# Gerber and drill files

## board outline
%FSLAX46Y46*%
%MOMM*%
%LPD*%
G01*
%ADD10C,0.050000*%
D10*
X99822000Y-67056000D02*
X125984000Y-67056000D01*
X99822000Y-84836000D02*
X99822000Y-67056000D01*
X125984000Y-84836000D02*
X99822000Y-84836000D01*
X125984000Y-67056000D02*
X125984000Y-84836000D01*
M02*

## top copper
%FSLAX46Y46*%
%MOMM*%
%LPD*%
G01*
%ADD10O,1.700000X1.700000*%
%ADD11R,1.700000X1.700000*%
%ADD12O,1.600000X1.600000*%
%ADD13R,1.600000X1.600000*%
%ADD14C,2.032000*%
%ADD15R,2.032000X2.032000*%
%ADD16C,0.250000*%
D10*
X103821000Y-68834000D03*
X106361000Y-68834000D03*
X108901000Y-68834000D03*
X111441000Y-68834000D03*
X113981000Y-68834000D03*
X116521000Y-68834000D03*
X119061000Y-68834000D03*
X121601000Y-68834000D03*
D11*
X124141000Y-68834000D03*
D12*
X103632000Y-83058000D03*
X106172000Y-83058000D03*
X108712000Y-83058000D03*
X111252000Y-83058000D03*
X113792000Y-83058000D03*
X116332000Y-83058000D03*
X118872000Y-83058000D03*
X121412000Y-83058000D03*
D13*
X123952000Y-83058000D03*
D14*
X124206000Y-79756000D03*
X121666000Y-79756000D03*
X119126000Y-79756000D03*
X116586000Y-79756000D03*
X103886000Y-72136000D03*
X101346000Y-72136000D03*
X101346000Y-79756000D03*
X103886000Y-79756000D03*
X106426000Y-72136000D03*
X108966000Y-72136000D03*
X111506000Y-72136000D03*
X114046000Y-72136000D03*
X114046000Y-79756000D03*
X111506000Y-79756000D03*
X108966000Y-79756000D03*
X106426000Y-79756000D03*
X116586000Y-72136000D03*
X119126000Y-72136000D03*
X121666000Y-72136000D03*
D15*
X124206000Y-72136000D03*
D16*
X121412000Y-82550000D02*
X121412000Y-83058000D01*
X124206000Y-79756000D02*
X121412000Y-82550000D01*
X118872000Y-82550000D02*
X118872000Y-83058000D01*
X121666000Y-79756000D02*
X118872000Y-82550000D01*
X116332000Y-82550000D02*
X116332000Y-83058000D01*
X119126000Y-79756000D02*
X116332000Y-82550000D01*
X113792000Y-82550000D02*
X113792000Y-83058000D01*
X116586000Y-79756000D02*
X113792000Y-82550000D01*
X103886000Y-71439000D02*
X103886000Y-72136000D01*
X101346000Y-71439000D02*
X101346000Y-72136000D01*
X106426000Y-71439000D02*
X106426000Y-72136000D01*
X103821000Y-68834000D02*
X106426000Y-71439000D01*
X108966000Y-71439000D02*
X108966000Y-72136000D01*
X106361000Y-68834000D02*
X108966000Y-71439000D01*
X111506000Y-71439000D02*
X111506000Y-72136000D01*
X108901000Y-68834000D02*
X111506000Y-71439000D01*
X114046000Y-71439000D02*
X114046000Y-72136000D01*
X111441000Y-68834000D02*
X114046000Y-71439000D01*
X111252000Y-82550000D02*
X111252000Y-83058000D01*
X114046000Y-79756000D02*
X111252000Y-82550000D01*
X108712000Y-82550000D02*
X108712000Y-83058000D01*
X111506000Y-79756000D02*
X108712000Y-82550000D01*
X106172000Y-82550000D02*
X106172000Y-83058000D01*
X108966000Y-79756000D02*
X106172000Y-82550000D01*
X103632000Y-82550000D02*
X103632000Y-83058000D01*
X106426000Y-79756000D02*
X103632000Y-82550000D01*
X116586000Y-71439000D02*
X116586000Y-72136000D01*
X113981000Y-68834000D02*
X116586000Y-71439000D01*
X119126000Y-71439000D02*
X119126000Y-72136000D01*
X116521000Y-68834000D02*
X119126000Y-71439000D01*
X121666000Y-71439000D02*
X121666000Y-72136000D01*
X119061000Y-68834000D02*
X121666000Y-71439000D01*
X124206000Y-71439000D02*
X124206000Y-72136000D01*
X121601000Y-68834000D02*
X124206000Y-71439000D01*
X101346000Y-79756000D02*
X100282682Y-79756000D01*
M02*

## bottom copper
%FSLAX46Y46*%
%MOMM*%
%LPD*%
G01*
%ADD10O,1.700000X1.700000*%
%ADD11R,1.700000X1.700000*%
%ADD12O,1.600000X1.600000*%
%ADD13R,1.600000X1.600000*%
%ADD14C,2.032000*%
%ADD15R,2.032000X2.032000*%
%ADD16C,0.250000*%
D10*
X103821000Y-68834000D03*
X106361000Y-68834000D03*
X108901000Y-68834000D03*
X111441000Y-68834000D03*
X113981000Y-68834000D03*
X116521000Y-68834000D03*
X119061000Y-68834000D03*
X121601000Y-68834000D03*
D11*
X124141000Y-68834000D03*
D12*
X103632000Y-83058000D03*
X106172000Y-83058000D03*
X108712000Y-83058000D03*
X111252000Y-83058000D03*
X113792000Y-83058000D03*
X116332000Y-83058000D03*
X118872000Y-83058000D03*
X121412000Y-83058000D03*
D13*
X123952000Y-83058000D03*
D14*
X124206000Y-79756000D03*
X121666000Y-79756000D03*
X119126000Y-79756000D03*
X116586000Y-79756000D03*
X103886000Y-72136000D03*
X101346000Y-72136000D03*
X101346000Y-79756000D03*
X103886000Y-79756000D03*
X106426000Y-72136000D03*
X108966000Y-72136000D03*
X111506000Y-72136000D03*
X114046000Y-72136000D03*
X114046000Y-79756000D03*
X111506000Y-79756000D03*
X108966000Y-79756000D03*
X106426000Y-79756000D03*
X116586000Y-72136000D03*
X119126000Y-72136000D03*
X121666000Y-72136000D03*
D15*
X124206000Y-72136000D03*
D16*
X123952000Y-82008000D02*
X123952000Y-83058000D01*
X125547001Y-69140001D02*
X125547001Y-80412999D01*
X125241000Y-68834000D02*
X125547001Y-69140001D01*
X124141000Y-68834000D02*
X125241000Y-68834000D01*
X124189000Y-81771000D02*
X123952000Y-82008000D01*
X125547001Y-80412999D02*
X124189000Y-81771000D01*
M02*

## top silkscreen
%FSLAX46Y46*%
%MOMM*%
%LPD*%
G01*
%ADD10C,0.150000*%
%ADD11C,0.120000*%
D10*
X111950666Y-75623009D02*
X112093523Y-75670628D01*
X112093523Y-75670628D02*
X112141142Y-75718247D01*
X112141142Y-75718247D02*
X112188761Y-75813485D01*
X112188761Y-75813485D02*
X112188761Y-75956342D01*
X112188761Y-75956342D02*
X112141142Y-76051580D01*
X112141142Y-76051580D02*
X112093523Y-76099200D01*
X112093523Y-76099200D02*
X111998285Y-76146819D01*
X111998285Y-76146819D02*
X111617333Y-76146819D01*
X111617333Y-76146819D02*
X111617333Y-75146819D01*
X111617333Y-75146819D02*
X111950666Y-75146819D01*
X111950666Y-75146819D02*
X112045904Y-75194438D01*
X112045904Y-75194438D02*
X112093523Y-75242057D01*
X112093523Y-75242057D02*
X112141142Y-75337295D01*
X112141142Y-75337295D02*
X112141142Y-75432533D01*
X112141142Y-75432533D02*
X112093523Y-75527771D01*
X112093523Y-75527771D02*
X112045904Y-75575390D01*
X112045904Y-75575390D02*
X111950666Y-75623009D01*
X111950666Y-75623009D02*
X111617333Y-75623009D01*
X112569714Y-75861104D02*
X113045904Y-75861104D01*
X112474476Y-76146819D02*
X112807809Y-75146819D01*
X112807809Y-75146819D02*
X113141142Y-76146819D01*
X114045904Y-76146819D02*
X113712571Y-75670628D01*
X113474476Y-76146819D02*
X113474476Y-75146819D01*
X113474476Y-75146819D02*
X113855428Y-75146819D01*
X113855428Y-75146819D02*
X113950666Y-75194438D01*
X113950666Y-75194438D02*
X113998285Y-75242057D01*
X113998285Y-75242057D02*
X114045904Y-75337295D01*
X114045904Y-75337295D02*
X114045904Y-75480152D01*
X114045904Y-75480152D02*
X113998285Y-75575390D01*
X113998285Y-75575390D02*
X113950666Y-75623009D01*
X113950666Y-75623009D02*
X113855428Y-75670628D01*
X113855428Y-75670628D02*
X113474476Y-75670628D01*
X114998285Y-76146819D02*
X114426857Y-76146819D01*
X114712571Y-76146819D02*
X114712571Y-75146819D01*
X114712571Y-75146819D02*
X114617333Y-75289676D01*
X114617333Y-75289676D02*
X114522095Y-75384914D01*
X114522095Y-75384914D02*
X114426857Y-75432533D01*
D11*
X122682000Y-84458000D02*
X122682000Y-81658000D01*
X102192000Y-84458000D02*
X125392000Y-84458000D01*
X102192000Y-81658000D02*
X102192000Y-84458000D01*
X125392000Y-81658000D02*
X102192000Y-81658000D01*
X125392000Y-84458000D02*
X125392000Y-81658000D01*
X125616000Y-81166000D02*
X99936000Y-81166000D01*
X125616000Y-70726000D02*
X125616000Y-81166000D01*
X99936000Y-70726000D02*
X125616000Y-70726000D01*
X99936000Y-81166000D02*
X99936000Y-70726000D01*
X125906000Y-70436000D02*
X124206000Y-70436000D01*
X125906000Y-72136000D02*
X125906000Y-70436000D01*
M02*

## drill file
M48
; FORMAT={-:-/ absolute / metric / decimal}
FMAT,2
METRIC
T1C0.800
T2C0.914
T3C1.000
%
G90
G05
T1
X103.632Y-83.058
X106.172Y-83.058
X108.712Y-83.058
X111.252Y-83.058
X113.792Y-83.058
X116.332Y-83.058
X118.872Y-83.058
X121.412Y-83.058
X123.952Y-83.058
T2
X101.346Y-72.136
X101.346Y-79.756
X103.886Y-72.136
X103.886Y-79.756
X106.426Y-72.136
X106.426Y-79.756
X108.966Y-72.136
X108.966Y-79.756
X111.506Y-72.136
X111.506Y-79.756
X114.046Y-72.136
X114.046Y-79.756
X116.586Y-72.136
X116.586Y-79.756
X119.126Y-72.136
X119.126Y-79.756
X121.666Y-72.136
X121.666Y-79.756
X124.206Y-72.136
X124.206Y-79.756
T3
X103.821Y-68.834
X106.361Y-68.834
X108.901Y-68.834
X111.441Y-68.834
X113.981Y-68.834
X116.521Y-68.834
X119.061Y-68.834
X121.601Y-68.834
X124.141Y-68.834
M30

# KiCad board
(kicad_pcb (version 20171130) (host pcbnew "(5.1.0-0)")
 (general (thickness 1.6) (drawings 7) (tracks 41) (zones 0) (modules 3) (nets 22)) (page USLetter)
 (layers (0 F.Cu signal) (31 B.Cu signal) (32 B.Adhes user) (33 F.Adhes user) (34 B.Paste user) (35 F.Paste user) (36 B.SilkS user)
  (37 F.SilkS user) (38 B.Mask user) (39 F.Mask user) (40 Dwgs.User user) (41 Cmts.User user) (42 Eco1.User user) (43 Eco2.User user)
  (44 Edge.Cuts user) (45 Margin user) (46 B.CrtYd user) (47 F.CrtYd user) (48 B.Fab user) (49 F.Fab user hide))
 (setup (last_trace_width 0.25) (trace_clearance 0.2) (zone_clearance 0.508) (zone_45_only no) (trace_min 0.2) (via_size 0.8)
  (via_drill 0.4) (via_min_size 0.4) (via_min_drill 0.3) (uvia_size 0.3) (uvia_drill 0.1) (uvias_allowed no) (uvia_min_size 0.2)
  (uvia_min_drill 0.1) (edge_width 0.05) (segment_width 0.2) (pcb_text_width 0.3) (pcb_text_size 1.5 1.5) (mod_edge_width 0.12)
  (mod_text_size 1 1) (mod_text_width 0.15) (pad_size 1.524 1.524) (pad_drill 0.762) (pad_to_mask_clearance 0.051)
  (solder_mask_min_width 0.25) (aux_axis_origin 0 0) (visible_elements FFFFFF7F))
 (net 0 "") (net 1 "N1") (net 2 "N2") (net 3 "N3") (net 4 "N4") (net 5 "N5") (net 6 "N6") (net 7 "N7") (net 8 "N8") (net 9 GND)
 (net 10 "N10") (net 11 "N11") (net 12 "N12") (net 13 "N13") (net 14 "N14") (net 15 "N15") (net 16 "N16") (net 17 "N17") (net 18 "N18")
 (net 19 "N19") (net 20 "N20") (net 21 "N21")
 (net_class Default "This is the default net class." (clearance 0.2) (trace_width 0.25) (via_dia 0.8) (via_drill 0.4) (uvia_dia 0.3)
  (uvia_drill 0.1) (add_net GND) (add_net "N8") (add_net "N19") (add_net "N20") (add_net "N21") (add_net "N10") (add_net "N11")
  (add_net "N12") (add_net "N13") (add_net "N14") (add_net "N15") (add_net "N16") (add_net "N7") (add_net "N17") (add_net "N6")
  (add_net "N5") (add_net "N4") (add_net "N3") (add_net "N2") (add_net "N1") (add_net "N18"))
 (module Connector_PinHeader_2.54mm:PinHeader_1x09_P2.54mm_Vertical (layer B.Cu) (at 124.141 68.834 90)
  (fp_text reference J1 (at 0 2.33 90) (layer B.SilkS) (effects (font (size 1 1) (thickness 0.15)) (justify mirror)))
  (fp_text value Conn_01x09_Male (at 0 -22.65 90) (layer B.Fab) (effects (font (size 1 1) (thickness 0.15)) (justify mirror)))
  (pad 9 thru_hole oval (at 0 -20.32 90) (size 1.7 1.7) (drill 1) (layers *.Cu *.Mask) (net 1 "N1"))
  (pad 8 thru_hole oval (at 0 -17.78 90) (size 1.7 1.7) (drill 1) (layers *.Cu *.Mask) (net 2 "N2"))
  (pad 7 thru_hole oval (at 0 -15.24 90) (size 1.7 1.7) (drill 1) (layers *.Cu *.Mask) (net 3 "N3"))
  (pad 6 thru_hole oval (at 0 -12.7 90) (size 1.7 1.7) (drill 1) (layers *.Cu *.Mask) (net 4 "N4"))
  (pad 5 thru_hole oval (at 0 -10.16 90) (size 1.7 1.7) (drill 1) (layers *.Cu *.Mask) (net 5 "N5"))
  (pad 4 thru_hole oval (at 0 -7.62 90) (size 1.7 1.7) (drill 1) (layers *.Cu *.Mask) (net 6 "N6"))
  (pad 3 thru_hole oval (at 0 -5.08 90) (size 1.7 1.7) (drill 1) (layers *.Cu *.Mask) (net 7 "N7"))
  (pad 2 thru_hole oval (at 0 -2.54 90) (size 1.7 1.7) (drill 1) (layers *.Cu *.Mask) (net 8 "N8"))
  (pad 1 thru_hole rect (at 0 0 90) (size 1.7 1.7) (drill 1) (layers *.Cu *.Mask) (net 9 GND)))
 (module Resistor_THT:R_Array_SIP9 (layer F.Cu) (at 123.952 83.058 180)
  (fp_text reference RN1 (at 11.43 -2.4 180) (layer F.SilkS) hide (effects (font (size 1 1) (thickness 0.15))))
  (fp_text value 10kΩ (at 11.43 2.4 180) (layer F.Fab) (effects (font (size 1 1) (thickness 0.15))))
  (fp_line (start 1.27 -1.4) (end 1.27 1.4) (layer F.SilkS) (width 0.12))
  (fp_line (start 21.76 -1.4) (end -1.44 -1.4) (layer F.SilkS) (width 0.12))
  (fp_line (start 21.76 1.4) (end 21.76 -1.4) (layer F.SilkS) (width 0.12))
  (fp_line (start -1.44 1.4) (end 21.76 1.4) (layer F.SilkS) (width 0.12))
  (fp_line (start -1.44 -1.4) (end -1.44 1.4) (layer F.SilkS) (width 0.12))
  (pad 9 thru_hole oval (at 20.32 0 180) (size 1.6 1.6) (drill 0.8) (layers *.Cu *.Mask) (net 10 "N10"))
  (pad 8 thru_hole oval (at 17.78 0 180) (size 1.6 1.6) (drill 0.8) (layers *.Cu *.Mask) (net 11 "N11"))
  (pad 7 thru_hole oval (at 15.24 0 180) (size 1.6 1.6) (drill 0.8) (layers *.Cu *.Mask) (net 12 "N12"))
  (pad 6 thru_hole oval (at 12.7 0 180) (size 1.6 1.6) (drill 0.8) (layers *.Cu *.Mask) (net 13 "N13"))
  (pad 5 thru_hole oval (at 10.16 0 180) (size 1.6 1.6) (drill 0.8) (layers *.Cu *.Mask) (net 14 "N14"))
  (pad 4 thru_hole oval (at 7.62 0 180) (size 1.6 1.6) (drill 0.8) (layers *.Cu *.Mask) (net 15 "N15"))
  (pad 3 thru_hole oval (at 5.08 0 180) (size 1.6 1.6) (drill 0.8) (layers *.Cu *.Mask) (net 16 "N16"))
  (pad 2 thru_hole oval (at 2.54 0 180) (size 1.6 1.6) (drill 0.8) (layers *.Cu *.Mask) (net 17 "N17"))
  (pad 1 thru_hole rect (at 0 0 180) (size 1.6 1.6) (drill 0.8) (layers *.Cu *.Mask) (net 9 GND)))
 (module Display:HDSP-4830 (layer F.Cu) (at 124.206 72.136 270)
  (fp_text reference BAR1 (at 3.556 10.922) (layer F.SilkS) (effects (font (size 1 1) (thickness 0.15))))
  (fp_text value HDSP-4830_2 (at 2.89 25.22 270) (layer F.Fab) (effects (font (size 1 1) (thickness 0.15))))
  (fp_line (start 9.03 -1.41) (end 9.03 24.27) (layer F.SilkS) (width 0.12))
  (fp_line (start -1.41 -1.41) (end 9.03 -1.41) (layer F.SilkS) (width 0.12))
  (fp_line (start -1.41 24.27) (end -1.41 -1.41) (layer F.SilkS) (width 0.12))
  (fp_line (start 9.03 24.27) (end -1.41 24.27) (layer F.SilkS) (width 0.12))
  (fp_line (start -1.7 -1.7) (end -1.7 0) (layer F.SilkS) (width 0.12))
  (fp_line (start 0 -1.7) (end -1.7 -1.7) (layer F.SilkS) (width 0.12))
  (pad 20 thru_hole circle (at 7.62 0 180) (size 2.032 2.032) (drill 0.9144) (layers *.Cu *.Mask) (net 17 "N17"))
  (pad 19 thru_hole circle (at 7.62 2.54 180) (size 2.032 2.032) (drill 0.9144) (layers *.Cu *.Mask) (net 16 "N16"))
  (pad 18 thru_hole circle (at 7.62 5.08 180) (size 2.032 2.032) (drill 0.9144) (layers *.Cu *.Mask) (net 15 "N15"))
  (pad 17 thru_hole circle (at 7.62 7.62 180) (size 2.032 2.032) (drill 0.9144) (layers *.Cu *.Mask) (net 14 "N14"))
  (pad 9 thru_hole circle (at 0 20.32 180) (size 2.032 2.032) (drill 0.9144) (layers *.Cu *.Mask) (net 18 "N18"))
  (pad 10 thru_hole circle (at 0 22.86 180) (size 2.032 2.032) (drill 0.9144) (layers *.Cu *.Mask) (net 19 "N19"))
  (pad 11 thru_hole circle (at 7.62 22.86 180) (size 2.032 2.032) (drill 0.9144) (layers *.Cu *.Mask) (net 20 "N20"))
  (pad 12 thru_hole circle (at 7.62 20.32 180) (size 2.032 2.032) (drill 0.9144) (layers *.Cu *.Mask) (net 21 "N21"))
  (pad 8 thru_hole circle (at 0 17.78 180) (size 2.032 2.032) (drill 0.9144) (layers *.Cu *.Mask) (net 1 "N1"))
  (pad 7 thru_hole circle (at 0 15.24 180) (size 2.032 2.032) (drill 0.9144) (layers *.Cu *.Mask) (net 2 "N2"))
  (pad 6 thru_hole circle (at 0 12.7 180) (size 2.032 2.032) (drill 0.9144) (layers *.Cu *.Mask) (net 3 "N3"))
  (pad 5 thru_hole circle (at 0 10.16 180) (size 2.032 2.032) (drill 0.9144) (layers *.Cu *.Mask) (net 4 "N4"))
  (pad 16 thru_hole circle (at 7.62 10.16 180) (size 2.032 2.032) (drill 0.9144) (layers *.Cu *.Mask) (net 13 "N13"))
  (pad 15 thru_hole circle (at 7.62 12.7 180) (size 2.032 2.032) (drill 0.9144) (layers *.Cu *.Mask) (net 12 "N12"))
  (pad 14 thru_hole circle (at 7.62 15.24 180) (size 2.032 2.032) (drill 0.9144) (layers *.Cu *.Mask) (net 11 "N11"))
  (pad 13 thru_hole circle (at 7.62 17.78 180) (size 2.032 2.032) (drill 0.9144) (layers *.Cu *.Mask) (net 10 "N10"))
  (pad 4 thru_hole circle (at 0 7.62 180) (size 2.032 2.032) (drill 0.9144) (layers *.Cu *.Mask) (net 5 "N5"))
  (pad 3 thru_hole circle (at 0 5.08 180) (size 2.032 2.032) (drill 0.9144) (layers *.Cu *.Mask) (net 6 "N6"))
  (pad 2 thru_hole circle (at 0 2.54 180) (size 2.032 2.032) (drill 0.9144) (layers *.Cu *.Mask) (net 7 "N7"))
  (pad 1 thru_hole rect (at 0 0 180) (size 2.032 2.032) (drill 0.9144) (layers *.Cu *.Mask) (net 8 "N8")))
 (gr_line (start 99.822 67.056) (end 125.984 67.056) (layer Edge.Cuts) (width 0.05))
 (gr_line (start 99.822 84.836) (end 99.822 67.056) (layer Edge.Cuts) (width 0.05))
 (gr_line (start 125.984 84.836) (end 99.822 84.836) (layer Edge.Cuts) (width 0.05))
 (gr_line (start 125.984 67.056) (end 125.984 84.836) (layer Edge.Cuts) (width 0.05))
 (segment (start 123.952 82.008) (end 123.952 83.058) (width 0.25) (layer B.Cu) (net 9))
 (segment (start 125.547001 69.140001) (end 125.547001 80.412999) (width 0.25) (layer B.Cu) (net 9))
 (segment (start 125.241 68.834) (end 125.547001 69.140001) (width 0.25) (layer B.Cu) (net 9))
 (segment (start 124.141 68.834) (end 125.241 68.834) (width 0.25) (layer B.Cu) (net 9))
 (segment (start 124.189 81.771) (end 123.952 82.008) (width 0.25) (layer B.Cu) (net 9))
 (segment (start 125.547001 80.412999) (end 124.189 81.771) (width 0.25) (layer B.Cu) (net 9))
 (segment (start 121.412 82.55) (end 121.412 83.058) (width 0.25) (layer F.Cu) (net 17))
 (segment (start 124.206 79.756) (end 121.412 82.55) (width 0.25) (layer F.Cu) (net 17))
 (segment (start 118.872 82.55) (end 118.872 83.058) (width 0.25) (layer F.Cu) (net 16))
 (segment (start 121.666 79.756) (end 118.872 82.55) (width 0.25) (layer F.Cu) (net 16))
 (segment (start 116.332 82.55) (end 116.332 83.058) (width 0.25) (layer F.Cu) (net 15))
 (segment (start 119.126 79.756) (end 116.332 82.55) (width 0.25) (layer F.Cu) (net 15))
 (segment (start 113.792 82.55) (end 113.792 83.058) (width 0.25) (layer F.Cu) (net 14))
 (segment (start 116.586 79.756) (end 113.792 82.55) (width 0.25) (layer F.Cu) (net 14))
 (segment (start 103.886 71.439) (end 103.886 72.136) (width 0.25) (layer F.Cu) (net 18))
 (segment (start 101.346 71.439) (end 101.346 72.136) (width 0.25) (layer F.Cu) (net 19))
 (segment (start 106.426 71.439) (end 106.426 72.136) (width 0.25) (layer F.Cu) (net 1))
 (segment (start 103.821 68.834) (end 106.426 71.439) (width 0.25) (layer F.Cu) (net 1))
 (segment (start 108.966 71.439) (end 108.966 72.136) (width 0.25) (layer F.Cu) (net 2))
 (segment (start 106.361 68.834) (end 108.966 71.439) (width 0.25) (layer F.Cu) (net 2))
 (segment (start 111.506 71.439) (end 111.506 72.136) (width 0.25) (layer F.Cu) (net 3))
 (segment (start 108.901 68.834) (end 111.506 71.439) (width 0.25) (layer F.Cu) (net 3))
 (segment (start 114.046 71.439) (end 114.046 72.136) (width 0.25) (layer F.Cu) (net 4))
 (segment (start 111.441 68.834) (end 114.046 71.439) (width 0.25) (layer F.Cu) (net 4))
 (segment (start 111.252 82.55) (end 111.252 83.058) (width 0.25) (layer F.Cu) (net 13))
 (segment (start 114.046 79.756) (end 111.252 82.55) (width 0.25) (layer F.Cu) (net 13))
 (segment (start 108.712 82.55) (end 108.712 83.058) (width 0.25) (layer F.Cu) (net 12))
 (segment (start 111.506 79.756) (end 108.712 82.55) (width 0.25) (layer F.Cu) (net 12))
 (segment (start 106.172 82.55) (end 106.172 83.058) (width 0.25) (layer F.Cu) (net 11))
 (segment (start 108.966 79.756) (end 106.172 82.55) (width 0.25) (layer F.Cu) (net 11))
 (segment (start 103.632 82.55) (end 103.632 83.058) (width 0.25) (layer F.Cu) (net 10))
 (segment (start 106.426 79.756) (end 103.632 82.55) (width 0.25) (layer F.Cu) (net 10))
 (segment (start 116.586 71.439) (end 116.586 72.136) (width 0.25) (layer F.Cu) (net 5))
 (segment (start 113.981 68.834) (end 116.586 71.439) (width 0.25) (layer F.Cu) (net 5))
 (segment (start 119.126 71.439) (end 119.126 72.136) (width 0.25) (layer F.Cu) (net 6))
 (segment (start 116.521 68.834) (end 119.126 71.439) (width 0.25) (layer F.Cu) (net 6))
 (segment (start 121.666 71.439) (end 121.666 72.136) (width 0.25) (layer F.Cu) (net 7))
 (segment (start 119.061 68.834) (end 121.666 71.439) (width 0.25) (layer F.Cu) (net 7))
 (segment (start 124.206 71.439) (end 124.206 72.136) (width 0.25) (layer F.Cu) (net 8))
 (segment (start 121.601 68.834) (end 124.206 71.439) (width 0.25) (layer F.Cu) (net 8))
 (segment (start 101.346 79.756) (end 100.282682 79.756) (width 0.25) (layer F.Cu) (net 20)))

